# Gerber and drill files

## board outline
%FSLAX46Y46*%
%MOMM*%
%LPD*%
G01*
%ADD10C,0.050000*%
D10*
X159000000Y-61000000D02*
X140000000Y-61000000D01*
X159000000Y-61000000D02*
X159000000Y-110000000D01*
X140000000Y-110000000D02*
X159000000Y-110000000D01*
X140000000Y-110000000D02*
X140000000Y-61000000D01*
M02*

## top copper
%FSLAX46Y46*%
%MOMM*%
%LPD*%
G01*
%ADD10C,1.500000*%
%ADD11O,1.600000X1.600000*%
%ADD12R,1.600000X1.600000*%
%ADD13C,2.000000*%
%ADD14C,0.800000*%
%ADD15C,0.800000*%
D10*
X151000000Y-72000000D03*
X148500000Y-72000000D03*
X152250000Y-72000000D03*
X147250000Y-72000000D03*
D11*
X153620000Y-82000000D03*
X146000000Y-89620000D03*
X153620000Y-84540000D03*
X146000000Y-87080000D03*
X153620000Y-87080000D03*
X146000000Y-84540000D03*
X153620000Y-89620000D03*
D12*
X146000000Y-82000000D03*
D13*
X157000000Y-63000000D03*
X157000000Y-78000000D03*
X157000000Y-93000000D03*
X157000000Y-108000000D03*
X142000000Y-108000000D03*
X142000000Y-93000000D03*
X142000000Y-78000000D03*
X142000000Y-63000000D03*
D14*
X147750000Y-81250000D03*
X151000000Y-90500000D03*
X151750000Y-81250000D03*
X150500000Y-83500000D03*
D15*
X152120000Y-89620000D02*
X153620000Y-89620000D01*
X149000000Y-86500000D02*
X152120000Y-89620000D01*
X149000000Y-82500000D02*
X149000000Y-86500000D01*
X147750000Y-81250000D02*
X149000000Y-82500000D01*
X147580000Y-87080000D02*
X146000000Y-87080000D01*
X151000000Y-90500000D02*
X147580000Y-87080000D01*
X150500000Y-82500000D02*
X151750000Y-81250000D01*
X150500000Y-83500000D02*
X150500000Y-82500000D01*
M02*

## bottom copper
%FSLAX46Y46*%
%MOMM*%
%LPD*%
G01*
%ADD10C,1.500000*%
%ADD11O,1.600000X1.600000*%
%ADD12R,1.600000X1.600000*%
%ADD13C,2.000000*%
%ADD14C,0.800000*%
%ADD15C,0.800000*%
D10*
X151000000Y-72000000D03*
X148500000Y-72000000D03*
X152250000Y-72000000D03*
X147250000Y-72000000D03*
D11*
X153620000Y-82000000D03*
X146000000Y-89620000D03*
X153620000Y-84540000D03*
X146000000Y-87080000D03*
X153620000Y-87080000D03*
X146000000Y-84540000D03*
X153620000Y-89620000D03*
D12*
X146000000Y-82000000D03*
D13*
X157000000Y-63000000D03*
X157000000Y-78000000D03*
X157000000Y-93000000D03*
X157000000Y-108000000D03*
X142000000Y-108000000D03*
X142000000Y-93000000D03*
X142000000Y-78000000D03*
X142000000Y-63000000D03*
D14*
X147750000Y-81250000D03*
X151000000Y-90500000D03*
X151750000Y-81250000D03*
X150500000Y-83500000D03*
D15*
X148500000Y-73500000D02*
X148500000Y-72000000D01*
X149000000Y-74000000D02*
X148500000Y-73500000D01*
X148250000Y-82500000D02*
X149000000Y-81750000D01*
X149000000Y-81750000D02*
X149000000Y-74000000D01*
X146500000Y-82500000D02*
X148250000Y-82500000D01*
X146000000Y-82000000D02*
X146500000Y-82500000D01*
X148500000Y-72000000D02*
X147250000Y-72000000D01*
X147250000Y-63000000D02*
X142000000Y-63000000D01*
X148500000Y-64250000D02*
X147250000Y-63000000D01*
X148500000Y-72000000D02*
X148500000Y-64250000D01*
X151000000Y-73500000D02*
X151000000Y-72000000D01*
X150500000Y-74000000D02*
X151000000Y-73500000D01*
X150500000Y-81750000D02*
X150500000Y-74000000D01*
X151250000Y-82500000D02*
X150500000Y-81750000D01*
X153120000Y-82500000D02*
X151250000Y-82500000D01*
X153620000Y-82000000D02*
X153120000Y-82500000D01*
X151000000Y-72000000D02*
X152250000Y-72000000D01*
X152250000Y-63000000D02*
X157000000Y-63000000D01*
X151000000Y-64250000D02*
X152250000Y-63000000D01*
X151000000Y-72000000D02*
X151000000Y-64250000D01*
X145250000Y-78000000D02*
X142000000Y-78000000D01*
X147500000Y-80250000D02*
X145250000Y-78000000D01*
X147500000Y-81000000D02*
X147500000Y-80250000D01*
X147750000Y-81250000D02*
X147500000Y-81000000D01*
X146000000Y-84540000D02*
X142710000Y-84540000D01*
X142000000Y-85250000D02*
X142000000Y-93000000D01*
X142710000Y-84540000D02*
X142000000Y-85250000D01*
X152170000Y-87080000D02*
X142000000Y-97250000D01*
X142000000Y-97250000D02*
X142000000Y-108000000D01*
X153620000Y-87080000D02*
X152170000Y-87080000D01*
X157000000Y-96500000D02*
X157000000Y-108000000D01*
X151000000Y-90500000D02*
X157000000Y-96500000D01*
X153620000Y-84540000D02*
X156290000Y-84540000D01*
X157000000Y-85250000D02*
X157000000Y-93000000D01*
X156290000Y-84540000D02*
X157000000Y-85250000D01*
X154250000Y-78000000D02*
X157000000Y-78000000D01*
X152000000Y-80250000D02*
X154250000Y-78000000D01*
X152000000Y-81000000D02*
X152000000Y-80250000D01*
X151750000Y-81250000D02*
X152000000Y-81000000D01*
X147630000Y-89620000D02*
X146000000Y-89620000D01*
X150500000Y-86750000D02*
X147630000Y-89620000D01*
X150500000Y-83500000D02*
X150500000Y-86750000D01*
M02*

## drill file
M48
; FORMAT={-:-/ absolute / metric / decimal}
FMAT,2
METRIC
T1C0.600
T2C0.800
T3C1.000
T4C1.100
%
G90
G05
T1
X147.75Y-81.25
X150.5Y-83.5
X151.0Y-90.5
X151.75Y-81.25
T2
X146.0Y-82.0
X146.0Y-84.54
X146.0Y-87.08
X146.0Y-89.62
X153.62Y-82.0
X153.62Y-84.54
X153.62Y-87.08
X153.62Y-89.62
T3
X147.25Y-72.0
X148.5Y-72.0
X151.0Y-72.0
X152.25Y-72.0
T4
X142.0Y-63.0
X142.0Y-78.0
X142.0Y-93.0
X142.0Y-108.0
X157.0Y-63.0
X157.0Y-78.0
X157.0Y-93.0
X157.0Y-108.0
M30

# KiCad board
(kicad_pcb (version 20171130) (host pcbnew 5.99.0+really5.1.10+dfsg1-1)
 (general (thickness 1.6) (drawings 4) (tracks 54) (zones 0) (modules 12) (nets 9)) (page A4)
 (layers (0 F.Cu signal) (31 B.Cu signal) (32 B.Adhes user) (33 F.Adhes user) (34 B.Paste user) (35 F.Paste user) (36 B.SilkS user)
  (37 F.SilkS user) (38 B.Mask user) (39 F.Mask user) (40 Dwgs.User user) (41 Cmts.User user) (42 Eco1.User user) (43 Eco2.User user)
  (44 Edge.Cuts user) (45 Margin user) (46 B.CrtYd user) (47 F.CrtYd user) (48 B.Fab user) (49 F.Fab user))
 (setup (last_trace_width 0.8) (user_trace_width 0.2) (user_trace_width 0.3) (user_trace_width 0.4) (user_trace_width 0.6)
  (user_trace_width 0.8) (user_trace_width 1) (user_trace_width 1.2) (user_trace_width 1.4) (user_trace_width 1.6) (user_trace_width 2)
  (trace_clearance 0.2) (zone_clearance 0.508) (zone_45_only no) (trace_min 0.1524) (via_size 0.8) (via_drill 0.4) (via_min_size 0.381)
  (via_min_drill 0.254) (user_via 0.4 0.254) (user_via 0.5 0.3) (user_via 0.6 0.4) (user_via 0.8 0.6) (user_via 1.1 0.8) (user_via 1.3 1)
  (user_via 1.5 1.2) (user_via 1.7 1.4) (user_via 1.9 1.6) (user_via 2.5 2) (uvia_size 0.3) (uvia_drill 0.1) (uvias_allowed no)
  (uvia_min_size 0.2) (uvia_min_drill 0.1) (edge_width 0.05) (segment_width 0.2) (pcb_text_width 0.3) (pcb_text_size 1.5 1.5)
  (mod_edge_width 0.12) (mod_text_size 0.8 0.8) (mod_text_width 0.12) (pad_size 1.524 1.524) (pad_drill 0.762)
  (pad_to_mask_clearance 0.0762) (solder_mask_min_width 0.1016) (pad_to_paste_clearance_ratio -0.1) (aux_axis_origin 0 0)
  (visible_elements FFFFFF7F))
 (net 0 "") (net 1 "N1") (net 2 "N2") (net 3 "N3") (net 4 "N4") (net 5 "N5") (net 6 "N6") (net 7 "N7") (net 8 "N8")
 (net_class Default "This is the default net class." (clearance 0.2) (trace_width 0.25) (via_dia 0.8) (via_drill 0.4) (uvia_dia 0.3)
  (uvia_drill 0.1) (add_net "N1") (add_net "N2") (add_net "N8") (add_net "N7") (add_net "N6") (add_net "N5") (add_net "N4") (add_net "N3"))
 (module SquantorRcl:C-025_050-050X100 (layer F.Cu) (at 149.75 72 180)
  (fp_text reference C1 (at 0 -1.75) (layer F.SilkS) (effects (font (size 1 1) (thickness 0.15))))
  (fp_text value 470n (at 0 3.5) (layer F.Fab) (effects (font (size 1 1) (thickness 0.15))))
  (pad 1 thru_hole circle (at -1.25 0 180) (size 1.5 1.5) (drill 1) (layers *.Cu *.Mask) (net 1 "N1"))
  (pad 2 thru_hole circle (at 1.25 0 180) (size 1.5 1.5) (drill 1) (layers *.Cu *.Mask) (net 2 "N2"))
  (pad 1 thru_hole circle (at -2.5 0 180) (size 1.5 1.5) (drill 1) (layers *.Cu *.Mask) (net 1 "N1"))
  (pad 2 thru_hole circle (at 2.5 0 180) (size 1.5 1.5) (drill 1) (layers *.Cu *.Mask) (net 2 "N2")))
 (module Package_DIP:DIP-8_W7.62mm (layer F.Cu) (at 146 82)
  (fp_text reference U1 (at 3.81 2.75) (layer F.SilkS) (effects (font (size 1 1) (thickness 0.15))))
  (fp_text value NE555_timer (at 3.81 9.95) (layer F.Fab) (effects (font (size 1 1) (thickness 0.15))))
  (pad 8 thru_hole oval (at 7.62 0) (size 1.6 1.6) (drill 0.8) (layers *.Cu *.Mask) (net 1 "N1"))
  (pad 4 thru_hole oval (at 0 7.62) (size 1.6 1.6) (drill 0.8) (layers *.Cu *.Mask) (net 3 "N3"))
  (pad 7 thru_hole oval (at 7.62 2.54) (size 1.6 1.6) (drill 0.8) (layers *.Cu *.Mask) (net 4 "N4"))
  (pad 3 thru_hole oval (at 0 5.08) (size 1.6 1.6) (drill 0.8) (layers *.Cu *.Mask) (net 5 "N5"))
  (pad 6 thru_hole oval (at 7.62 5.08) (size 1.6 1.6) (drill 0.8) (layers *.Cu *.Mask) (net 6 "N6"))
  (pad 2 thru_hole oval (at 0 2.54) (size 1.6 1.6) (drill 0.8) (layers *.Cu *.Mask) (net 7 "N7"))
  (pad 5 thru_hole oval (at 7.62 7.62) (size 1.6 1.6) (drill 0.8) (layers *.Cu *.Mask) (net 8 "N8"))
  (pad 1 thru_hole rect (at 0 0) (size 1.6 1.6) (drill 0.8) (layers *.Cu *.Mask) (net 2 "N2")))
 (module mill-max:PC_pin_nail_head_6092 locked (layer F.Cu) (at 157 63)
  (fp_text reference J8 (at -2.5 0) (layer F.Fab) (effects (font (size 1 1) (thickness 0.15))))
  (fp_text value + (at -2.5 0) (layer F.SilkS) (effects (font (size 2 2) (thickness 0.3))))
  (pad 1 thru_hole circle (at 0 0) (size 2 2) (drill 1.1) (layers *.Cu *.Mask) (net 1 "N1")))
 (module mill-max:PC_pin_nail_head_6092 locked (layer F.Cu) (at 157 78)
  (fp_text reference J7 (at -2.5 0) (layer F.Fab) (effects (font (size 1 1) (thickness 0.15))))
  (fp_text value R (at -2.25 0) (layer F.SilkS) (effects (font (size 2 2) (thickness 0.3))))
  (pad 1 thru_hole circle (at 0 0) (size 2 2) (drill 1.1) (layers *.Cu *.Mask) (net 3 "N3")))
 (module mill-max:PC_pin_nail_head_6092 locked (layer F.Cu) (at 157 93)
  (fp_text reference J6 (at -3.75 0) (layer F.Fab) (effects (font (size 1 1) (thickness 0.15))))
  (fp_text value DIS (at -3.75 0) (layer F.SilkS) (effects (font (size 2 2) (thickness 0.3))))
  (pad 1 thru_hole circle (at 0 0) (size 2 2) (drill 1.1) (layers *.Cu *.Mask) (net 4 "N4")))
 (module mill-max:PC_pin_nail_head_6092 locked (layer F.Cu) (at 157 108)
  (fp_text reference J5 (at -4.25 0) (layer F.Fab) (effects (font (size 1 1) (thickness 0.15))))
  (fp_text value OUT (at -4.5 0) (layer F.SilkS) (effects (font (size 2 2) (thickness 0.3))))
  (pad 1 thru_hole circle (at 0 0) (size 2 2) (drill 1.1) (layers *.Cu *.Mask) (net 5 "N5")))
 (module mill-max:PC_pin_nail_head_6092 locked (layer F.Cu) (at 142 108)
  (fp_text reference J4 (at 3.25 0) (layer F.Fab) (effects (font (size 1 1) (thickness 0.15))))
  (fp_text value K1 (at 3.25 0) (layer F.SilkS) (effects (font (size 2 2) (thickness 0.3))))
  (pad 1 thru_hole circle (at 0 0) (size 2 2) (drill 1.1) (layers *.Cu *.Mask) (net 6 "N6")))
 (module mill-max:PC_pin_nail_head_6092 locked (layer F.Cu) (at 142 93)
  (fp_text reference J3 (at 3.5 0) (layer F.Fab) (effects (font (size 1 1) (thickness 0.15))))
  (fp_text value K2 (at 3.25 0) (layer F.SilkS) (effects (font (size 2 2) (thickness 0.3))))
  (pad 1 thru_hole circle (at 0 0) (size 2 2) (drill 1.1) (layers *.Cu *.Mask) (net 7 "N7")))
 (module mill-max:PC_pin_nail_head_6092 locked (layer F.Cu) (at 142 78)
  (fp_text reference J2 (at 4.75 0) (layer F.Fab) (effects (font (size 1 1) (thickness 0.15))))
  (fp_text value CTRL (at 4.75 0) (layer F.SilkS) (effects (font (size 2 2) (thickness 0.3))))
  (pad 1 thru_hole circle (at 0 0) (size 2 2) (drill 1.1) (layers *.Cu *.Mask) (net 8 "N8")))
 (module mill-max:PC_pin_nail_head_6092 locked (layer F.Cu) (at 142 63)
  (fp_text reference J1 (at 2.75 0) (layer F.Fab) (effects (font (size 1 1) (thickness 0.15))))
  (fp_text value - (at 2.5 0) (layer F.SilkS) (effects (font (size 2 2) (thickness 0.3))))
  (pad 1 thru_hole circle (at 0 0) (size 2 2) (drill 1.1) (layers *.Cu *.Mask) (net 2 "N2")))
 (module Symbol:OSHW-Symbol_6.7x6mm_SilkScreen (layer B.Cu) (at 150 99.5 180)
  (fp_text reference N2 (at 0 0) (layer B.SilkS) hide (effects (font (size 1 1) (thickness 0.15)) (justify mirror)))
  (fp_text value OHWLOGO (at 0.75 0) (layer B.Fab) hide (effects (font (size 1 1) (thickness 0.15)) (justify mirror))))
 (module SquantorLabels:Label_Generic (layer B.Cu) (at 149 103.5)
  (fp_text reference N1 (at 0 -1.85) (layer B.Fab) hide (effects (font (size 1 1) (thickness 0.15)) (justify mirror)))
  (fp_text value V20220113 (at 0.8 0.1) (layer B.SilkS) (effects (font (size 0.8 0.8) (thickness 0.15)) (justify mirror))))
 (gr_line (start 159 61) (end 140 61) (layer Edge.Cuts) (width 0.05))
 (gr_line (start 159 61) (end 159 110) (layer Edge.Cuts) (width 0.05))
 (gr_line (start 140 110) (end 159 110) (layer Edge.Cuts) (width 0.05))
 (gr_line (start 140 110) (end 140 61) (layer Edge.Cuts) (width 0.05))
 (segment (start 148.5 73.5) (end 148.5 72) (width 0.8) (layer B.Cu) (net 2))
 (segment (start 149 74) (end 148.5 73.5) (width 0.8) (layer B.Cu) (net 2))
 (segment (start 148.25 82.5) (end 149 81.75) (width 0.8) (layer B.Cu) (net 2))
 (segment (start 149 81.75) (end 149 74) (width 0.8) (layer B.Cu) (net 2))
 (segment (start 146.5 82.5) (end 148.25 82.5) (width 0.8) (layer B.Cu) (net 2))
 (segment (start 146 82) (end 146.5 82.5) (width 0.8) (layer B.Cu) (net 2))
 (segment (start 148.5 72) (end 147.25 72) (width 0.8) (layer B.Cu) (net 2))
 (segment (start 147.25 63) (end 142 63) (width 0.8) (layer B.Cu) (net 2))
 (segment (start 148.5 64.25) (end 147.25 63) (width 0.8) (layer B.Cu) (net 2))
 (segment (start 148.5 72) (end 148.5 64.25) (width 0.8) (layer B.Cu) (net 2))
 (segment (start 151 73.5) (end 151 72) (width 0.8) (layer B.Cu) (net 1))
 (segment (start 150.5 74) (end 151 73.5) (width 0.8) (layer B.Cu) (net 1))
 (segment (start 150.5 81.75) (end 150.5 74) (width 0.8) (layer B.Cu) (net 1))
 (segment (start 151.25 82.5) (end 150.5 81.75) (width 0.8) (layer B.Cu) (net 1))
 (segment (start 153.12 82.5) (end 151.25 82.5) (width 0.8) (layer B.Cu) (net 1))
 (segment (start 153.62 82) (end 153.12 82.5) (width 0.8) (layer B.Cu) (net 1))
 (segment (start 151 72) (end 152.25 72) (width 0.8) (layer B.Cu) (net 1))
 (segment (start 152.25 63) (end 157 63) (width 0.8) (layer B.Cu) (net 1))
 (segment (start 151 64.25) (end 152.25 63) (width 0.8) (layer B.Cu) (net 1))
 (segment (start 151 72) (end 151 64.25) (width 0.8) (layer B.Cu) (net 1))
 (via (at 147.75 81.25) (size 0.8) (drill 0.6) (layers F.Cu B.Cu) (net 8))
 (segment (start 145.25 78) (end 142 78) (width 0.8) (layer B.Cu) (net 8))
 (segment (start 147.5 80.25) (end 145.25 78) (width 0.8) (layer B.Cu) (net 8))
 (segment (start 147.5 81) (end 147.5 80.25) (width 0.8) (layer B.Cu) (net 8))
 (segment (start 147.75 81.25) (end 147.5 81) (width 0.8) (layer B.Cu) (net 8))
 (segment (start 152.12 89.62) (end 153.62 89.62) (width 0.8) (layer F.Cu) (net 8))
 (segment (start 149 86.5) (end 152.12 89.62) (width 0.8) (layer F.Cu) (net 8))
 (segment (start 149 82.5) (end 149 86.5) (width 0.8) (layer F.Cu) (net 8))
 (segment (start 147.75 81.25) (end 149 82.5) (width 0.8) (layer F.Cu) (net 8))
 (segment (start 146 84.54) (end 142.71 84.54) (width 0.8) (layer B.Cu) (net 7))
 (segment (start 142 85.25) (end 142 93) (width 0.8) (layer B.Cu) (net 7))
 (segment (start 142.71 84.54) (end 142 85.25) (width 0.8) (layer B.Cu) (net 7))
 (segment (start 152.17 87.08) (end 142 97.25) (width 0.8) (layer B.Cu) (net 6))
 (segment (start 142 97.25) (end 142 108) (width 0.8) (layer B.Cu) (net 6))
 (segment (start 153.62 87.08) (end 152.17 87.08) (width 0.8) (layer B.Cu) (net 6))
 (segment (start 147.58 87.08) (end 146 87.08) (width 0.8) (layer F.Cu) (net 5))
 (segment (start 151 90.5) (end 147.58 87.08) (width 0.8) (layer F.Cu) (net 5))
 (via (at 151 90.5) (size 0.8) (drill 0.6) (layers F.Cu B.Cu) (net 5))
 (segment (start 157 96.5) (end 157 108) (width 0.8) (layer B.Cu) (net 5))
 (segment (start 151 90.5) (end 157 96.5) (width 0.8) (layer B.Cu) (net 5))
 (segment (start 153.62 84.54) (end 156.29 84.54) (width 0.8) (layer B.Cu) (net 4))
 (segment (start 157 85.25) (end 157 93) (width 0.8) (layer B.Cu) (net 4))
 (segment (start 156.29 84.54) (end 157 85.25) (width 0.8) (layer B.Cu) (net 4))
 (via (at 151.75 81.25) (size 0.8) (drill 0.6) (layers F.Cu B.Cu) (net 3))
 (segment (start 154.25 78) (end 157 78) (width 0.8) (layer B.Cu) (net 3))
 (segment (start 152 80.25) (end 154.25 78) (width 0.8) (layer B.Cu) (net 3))
 (segment (start 152 81) (end 152 80.25) (width 0.8) (layer B.Cu) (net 3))
 (segment (start 151.75 81.25) (end 152 81) (width 0.8) (layer B.Cu) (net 3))
 (segment (start 147.63 89.62) (end 146 89.62) (width 0.8) (layer B.Cu) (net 3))
 (segment (start 150.5 86.75) (end 147.63 89.62) (width 0.8) (layer B.Cu) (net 3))
 (segment (start 150.5 83.5) (end 150.5 86.75) (width 0.8) (layer B.Cu) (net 3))
 (segment (start 150.5 82.5) (end 151.75 81.25) (width 0.8) (layer F.Cu) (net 3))
 (segment (start 150.5 83.5) (end 150.5 82.5) (width 0.8) (layer F.Cu) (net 3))
 (via (at 150.5 83.5) (size 0.8) (drill 0.6) (layers F.Cu B.Cu) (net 3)))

